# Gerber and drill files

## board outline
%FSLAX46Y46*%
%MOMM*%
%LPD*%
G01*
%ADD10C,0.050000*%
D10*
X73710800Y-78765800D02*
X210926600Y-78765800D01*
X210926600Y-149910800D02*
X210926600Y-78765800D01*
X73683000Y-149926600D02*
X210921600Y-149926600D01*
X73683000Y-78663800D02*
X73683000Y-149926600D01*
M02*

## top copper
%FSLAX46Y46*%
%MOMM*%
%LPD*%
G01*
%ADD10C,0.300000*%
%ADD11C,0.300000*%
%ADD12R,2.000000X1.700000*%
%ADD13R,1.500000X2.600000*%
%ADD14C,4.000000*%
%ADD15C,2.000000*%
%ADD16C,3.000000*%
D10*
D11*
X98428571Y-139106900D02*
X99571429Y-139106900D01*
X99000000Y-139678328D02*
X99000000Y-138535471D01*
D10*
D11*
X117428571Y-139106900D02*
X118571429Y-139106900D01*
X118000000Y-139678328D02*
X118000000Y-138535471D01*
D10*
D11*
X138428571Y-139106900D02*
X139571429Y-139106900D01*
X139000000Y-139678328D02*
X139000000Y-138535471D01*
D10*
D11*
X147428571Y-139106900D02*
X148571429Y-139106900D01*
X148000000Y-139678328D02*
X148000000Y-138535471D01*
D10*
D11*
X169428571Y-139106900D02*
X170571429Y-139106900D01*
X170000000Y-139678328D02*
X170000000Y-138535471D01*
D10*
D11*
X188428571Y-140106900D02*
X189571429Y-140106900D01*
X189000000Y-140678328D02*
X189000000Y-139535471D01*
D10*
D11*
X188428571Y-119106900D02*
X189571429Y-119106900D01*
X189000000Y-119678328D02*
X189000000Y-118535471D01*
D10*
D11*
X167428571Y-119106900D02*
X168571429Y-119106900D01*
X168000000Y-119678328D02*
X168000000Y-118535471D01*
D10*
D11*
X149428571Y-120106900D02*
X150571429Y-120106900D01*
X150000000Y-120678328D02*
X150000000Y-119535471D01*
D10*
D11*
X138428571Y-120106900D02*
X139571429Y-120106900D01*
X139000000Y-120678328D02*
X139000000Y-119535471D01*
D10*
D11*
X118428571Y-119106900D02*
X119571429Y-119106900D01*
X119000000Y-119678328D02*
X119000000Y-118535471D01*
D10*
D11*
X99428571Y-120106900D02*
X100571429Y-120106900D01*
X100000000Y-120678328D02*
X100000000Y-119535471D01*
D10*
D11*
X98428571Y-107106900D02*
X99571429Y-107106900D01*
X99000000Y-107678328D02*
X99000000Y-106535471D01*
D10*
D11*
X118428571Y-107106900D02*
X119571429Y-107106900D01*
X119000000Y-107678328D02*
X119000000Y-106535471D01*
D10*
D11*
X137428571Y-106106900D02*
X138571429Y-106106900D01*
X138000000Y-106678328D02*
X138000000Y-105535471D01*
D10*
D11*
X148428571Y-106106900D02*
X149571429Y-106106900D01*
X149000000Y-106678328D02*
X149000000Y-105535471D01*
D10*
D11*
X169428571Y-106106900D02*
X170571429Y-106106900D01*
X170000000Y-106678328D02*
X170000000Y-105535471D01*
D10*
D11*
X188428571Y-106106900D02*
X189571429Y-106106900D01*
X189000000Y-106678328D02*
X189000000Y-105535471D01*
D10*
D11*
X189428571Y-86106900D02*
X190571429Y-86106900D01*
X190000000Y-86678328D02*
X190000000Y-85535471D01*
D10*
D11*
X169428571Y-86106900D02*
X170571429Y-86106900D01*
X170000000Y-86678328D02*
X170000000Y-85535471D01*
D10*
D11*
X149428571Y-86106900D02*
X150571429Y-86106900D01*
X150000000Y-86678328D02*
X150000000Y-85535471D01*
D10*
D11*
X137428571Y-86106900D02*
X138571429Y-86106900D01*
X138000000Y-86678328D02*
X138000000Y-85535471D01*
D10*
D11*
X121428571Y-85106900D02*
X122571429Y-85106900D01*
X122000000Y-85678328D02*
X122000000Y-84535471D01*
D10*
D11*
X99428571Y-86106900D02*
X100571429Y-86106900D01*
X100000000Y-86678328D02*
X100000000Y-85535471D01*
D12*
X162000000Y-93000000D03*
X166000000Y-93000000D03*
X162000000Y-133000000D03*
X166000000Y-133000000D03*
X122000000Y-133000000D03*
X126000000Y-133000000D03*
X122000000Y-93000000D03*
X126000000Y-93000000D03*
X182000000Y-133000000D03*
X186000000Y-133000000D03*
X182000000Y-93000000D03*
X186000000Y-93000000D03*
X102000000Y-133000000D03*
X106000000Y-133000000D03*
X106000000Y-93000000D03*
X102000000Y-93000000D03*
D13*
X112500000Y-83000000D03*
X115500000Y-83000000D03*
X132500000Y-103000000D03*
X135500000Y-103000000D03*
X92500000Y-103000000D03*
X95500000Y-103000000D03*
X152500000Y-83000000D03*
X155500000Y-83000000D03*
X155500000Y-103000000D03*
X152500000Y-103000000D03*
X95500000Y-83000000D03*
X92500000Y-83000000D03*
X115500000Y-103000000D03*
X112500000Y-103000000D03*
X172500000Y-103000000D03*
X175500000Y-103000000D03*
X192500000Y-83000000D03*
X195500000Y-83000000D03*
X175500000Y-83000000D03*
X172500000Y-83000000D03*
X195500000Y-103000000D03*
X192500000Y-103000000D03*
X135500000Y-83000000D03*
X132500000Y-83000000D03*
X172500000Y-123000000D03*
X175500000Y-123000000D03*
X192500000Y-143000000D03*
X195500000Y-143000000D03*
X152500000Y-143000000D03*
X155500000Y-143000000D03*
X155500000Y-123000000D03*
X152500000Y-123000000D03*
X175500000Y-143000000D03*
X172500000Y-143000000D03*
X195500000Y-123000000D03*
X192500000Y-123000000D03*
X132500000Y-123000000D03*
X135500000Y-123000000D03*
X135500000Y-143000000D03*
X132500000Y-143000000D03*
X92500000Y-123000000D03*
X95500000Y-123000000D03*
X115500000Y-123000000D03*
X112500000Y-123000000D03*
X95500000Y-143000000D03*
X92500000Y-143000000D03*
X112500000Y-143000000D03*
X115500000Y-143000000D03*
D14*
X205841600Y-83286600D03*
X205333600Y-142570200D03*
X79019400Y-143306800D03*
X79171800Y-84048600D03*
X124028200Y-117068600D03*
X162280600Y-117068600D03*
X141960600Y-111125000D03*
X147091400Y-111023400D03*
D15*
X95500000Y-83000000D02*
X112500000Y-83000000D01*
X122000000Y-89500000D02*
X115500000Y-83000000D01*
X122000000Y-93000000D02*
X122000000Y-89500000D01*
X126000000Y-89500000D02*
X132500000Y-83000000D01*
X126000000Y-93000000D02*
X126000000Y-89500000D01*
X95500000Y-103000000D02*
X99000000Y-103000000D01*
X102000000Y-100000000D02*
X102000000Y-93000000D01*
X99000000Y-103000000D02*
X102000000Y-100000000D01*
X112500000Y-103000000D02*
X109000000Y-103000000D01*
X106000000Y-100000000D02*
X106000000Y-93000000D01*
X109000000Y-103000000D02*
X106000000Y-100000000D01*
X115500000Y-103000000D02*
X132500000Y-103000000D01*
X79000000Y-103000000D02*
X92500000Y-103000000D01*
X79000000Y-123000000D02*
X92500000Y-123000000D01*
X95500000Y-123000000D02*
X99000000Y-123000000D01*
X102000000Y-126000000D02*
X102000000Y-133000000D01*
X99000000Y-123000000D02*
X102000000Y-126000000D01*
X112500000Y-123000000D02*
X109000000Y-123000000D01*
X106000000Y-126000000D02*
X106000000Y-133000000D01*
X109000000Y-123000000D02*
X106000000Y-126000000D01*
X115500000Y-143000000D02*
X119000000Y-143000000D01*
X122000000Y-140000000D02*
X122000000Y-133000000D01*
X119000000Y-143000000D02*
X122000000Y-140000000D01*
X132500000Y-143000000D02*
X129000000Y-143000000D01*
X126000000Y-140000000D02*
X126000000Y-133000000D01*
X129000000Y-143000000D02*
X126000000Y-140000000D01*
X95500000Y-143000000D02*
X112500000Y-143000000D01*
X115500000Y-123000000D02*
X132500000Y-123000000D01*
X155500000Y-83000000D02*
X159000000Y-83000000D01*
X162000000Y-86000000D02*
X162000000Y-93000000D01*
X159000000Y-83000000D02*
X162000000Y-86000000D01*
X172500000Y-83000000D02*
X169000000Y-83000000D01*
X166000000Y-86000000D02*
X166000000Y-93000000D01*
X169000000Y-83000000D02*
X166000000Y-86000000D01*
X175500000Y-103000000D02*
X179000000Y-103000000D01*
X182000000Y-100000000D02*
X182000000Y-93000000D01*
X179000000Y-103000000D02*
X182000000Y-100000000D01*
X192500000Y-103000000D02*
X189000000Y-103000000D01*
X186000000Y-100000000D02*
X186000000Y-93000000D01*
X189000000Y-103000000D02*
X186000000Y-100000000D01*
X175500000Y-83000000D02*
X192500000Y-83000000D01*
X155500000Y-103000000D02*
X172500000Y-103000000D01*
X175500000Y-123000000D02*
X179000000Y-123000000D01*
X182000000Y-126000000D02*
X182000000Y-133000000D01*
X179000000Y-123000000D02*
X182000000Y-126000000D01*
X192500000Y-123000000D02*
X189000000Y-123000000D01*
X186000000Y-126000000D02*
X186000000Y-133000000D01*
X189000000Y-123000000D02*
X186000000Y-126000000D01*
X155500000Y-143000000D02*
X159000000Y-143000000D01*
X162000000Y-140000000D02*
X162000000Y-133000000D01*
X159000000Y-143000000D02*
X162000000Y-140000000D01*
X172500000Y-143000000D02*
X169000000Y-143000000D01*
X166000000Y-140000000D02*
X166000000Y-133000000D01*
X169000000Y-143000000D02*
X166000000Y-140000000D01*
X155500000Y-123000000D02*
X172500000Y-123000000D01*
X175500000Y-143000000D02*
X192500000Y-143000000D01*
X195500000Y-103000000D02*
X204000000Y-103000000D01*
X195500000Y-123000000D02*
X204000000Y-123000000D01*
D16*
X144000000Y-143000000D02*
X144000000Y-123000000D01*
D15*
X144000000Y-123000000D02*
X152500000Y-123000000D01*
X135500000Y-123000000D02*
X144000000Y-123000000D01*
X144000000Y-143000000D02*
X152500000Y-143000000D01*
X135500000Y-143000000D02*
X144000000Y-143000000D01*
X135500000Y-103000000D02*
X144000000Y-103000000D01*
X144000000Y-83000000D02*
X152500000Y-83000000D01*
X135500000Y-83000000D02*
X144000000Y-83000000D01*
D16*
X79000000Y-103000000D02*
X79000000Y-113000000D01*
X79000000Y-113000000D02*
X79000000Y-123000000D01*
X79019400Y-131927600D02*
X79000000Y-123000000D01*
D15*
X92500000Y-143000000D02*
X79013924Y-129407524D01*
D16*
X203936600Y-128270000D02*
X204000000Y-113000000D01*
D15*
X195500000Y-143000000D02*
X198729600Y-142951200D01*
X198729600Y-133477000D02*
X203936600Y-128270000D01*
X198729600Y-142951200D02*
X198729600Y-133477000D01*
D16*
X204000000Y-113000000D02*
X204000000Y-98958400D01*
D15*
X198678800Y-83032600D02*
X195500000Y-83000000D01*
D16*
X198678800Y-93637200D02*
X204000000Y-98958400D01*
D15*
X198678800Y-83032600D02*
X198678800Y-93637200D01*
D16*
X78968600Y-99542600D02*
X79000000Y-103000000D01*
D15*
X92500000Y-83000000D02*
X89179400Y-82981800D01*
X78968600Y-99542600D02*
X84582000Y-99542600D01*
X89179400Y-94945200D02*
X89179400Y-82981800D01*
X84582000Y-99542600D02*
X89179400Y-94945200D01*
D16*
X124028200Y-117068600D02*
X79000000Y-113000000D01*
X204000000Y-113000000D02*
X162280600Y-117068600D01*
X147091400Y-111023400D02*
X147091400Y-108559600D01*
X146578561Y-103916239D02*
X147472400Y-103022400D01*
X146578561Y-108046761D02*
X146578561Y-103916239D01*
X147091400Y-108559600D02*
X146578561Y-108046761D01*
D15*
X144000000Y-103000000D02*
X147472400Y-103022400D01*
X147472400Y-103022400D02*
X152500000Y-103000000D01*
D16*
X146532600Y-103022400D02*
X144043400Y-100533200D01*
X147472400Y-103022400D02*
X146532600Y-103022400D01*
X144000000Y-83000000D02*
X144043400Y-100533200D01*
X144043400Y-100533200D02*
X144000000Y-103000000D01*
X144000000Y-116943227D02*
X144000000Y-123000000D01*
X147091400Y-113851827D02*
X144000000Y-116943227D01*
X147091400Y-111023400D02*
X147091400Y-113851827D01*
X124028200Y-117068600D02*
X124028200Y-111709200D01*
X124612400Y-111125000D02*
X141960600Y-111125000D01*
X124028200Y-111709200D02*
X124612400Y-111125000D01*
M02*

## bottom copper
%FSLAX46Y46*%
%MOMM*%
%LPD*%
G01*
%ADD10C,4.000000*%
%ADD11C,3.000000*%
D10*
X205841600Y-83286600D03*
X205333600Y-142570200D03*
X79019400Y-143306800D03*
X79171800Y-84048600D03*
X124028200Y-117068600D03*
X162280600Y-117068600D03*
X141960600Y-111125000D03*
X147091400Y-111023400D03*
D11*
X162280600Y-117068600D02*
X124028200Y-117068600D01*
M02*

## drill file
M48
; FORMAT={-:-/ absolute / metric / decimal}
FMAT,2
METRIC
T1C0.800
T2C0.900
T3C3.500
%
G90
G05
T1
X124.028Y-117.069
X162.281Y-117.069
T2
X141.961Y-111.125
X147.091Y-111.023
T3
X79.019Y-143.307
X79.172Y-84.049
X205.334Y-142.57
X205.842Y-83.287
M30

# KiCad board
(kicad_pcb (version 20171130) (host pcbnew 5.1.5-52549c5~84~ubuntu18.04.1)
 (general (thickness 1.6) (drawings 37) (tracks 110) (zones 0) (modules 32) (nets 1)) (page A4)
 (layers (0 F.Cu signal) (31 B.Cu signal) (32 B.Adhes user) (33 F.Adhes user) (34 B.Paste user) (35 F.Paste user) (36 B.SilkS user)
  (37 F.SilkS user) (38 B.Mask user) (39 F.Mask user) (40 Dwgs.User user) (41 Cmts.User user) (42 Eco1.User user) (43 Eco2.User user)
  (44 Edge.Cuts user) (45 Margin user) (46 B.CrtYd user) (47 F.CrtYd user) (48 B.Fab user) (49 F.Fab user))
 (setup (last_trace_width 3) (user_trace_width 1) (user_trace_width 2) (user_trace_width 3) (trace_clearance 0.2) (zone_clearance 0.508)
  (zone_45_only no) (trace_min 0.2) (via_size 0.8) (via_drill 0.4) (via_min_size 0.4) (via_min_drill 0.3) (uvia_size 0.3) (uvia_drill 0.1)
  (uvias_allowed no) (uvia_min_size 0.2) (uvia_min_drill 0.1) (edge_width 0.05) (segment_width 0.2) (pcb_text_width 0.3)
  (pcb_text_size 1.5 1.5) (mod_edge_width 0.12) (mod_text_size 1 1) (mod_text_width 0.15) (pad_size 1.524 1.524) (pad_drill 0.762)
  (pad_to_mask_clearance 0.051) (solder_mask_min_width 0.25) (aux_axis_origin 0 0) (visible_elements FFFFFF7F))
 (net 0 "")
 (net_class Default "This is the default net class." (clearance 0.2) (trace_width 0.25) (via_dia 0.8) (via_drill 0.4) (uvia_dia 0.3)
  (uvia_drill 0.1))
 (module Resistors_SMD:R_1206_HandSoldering (layer F.Cu) (at 164 93)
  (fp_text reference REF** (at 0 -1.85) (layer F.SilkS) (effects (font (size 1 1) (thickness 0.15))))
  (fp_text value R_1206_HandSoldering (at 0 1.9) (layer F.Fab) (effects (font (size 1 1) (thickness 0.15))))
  (pad 1 smd rect (at -2 0) (size 2 1.7) (layers F.Cu F.Paste F.Mask))
  (pad 2 smd rect (at 2 0) (size 2 1.7) (layers F.Cu F.Paste F.Mask)))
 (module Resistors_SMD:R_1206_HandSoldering (layer F.Cu) (at 164 133)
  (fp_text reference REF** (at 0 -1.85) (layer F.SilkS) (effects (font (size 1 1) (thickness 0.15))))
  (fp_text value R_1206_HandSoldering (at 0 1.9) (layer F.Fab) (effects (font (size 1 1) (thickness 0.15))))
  (pad 1 smd rect (at -2 0) (size 2 1.7) (layers F.Cu F.Paste F.Mask))
  (pad 2 smd rect (at 2 0) (size 2 1.7) (layers F.Cu F.Paste F.Mask)))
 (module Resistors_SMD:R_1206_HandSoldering (layer F.Cu) (at 124 133)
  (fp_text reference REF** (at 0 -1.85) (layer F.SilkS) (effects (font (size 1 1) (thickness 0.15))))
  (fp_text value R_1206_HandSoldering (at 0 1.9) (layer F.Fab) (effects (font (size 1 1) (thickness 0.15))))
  (pad 1 smd rect (at -2 0) (size 2 1.7) (layers F.Cu F.Paste F.Mask))
  (pad 2 smd rect (at 2 0) (size 2 1.7) (layers F.Cu F.Paste F.Mask)))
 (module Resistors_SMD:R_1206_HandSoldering (layer F.Cu) (at 124 93)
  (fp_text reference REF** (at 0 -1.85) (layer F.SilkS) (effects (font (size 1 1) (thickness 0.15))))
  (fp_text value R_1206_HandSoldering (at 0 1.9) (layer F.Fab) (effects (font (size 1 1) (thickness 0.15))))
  (pad 1 smd rect (at -2 0) (size 2 1.7) (layers F.Cu F.Paste F.Mask))
  (pad 2 smd rect (at 2 0) (size 2 1.7) (layers F.Cu F.Paste F.Mask)))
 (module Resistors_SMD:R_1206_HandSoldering (layer F.Cu) (at 184 133)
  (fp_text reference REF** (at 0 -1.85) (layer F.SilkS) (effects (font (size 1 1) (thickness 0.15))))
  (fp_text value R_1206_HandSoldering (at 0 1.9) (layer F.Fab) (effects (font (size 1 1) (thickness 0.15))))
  (pad 1 smd rect (at -2 0) (size 2 1.7) (layers F.Cu F.Paste F.Mask))
  (pad 2 smd rect (at 2 0) (size 2 1.7) (layers F.Cu F.Paste F.Mask)))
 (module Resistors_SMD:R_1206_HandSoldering (layer F.Cu) (at 184 93)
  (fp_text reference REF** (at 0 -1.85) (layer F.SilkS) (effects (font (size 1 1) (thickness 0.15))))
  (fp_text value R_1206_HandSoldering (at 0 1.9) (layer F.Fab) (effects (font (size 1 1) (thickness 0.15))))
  (pad 1 smd rect (at -2 0) (size 2 1.7) (layers F.Cu F.Paste F.Mask))
  (pad 2 smd rect (at 2 0) (size 2 1.7) (layers F.Cu F.Paste F.Mask)))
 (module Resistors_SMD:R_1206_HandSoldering (layer F.Cu) (at 104 133)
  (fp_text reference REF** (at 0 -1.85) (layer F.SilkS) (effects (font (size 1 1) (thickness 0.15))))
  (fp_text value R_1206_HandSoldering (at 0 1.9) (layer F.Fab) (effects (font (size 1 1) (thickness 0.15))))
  (pad 1 smd rect (at -2 0) (size 2 1.7) (layers F.Cu F.Paste F.Mask))
  (pad 2 smd rect (at 2 0) (size 2 1.7) (layers F.Cu F.Paste F.Mask)))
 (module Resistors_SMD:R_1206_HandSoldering (layer F.Cu) (at 104 93)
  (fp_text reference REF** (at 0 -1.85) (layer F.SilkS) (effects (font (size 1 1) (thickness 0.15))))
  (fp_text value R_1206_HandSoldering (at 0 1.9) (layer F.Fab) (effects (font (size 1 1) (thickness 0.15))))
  (pad 2 smd rect (at 2 0) (size 2 1.7) (layers F.Cu F.Paste F.Mask))
  (pad 1 smd rect (at -2 0) (size 2 1.7) (layers F.Cu F.Paste F.Mask)))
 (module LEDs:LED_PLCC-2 (layer F.Cu) (at 114 83 180)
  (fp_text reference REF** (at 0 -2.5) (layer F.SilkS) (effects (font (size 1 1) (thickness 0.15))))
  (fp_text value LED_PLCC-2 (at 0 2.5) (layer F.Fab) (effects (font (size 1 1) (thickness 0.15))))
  (pad 2 smd rect (at 1.5 0 180) (size 1.5 2.6) (layers F.Cu F.Paste F.Mask))
  (pad 1 smd rect (at -1.5 0 180) (size 1.5 2.6) (layers F.Cu F.Paste F.Mask)))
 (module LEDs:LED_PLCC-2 (layer F.Cu) (at 134 103 180)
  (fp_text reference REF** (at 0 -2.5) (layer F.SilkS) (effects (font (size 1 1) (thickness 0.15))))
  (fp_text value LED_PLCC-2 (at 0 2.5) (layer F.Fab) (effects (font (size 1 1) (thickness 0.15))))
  (pad 2 smd rect (at 1.5 0 180) (size 1.5 2.6) (layers F.Cu F.Paste F.Mask))
  (pad 1 smd rect (at -1.5 0 180) (size 1.5 2.6) (layers F.Cu F.Paste F.Mask)))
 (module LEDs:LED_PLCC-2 (layer F.Cu) (at 94 103 180)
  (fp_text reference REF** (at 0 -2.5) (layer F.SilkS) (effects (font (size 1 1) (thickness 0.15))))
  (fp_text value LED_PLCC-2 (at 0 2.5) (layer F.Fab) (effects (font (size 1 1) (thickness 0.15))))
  (pad 2 smd rect (at 1.5 0 180) (size 1.5 2.6) (layers F.Cu F.Paste F.Mask))
  (pad 1 smd rect (at -1.5 0 180) (size 1.5 2.6) (layers F.Cu F.Paste F.Mask)))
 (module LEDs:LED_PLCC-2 (layer F.Cu) (at 154 83 180)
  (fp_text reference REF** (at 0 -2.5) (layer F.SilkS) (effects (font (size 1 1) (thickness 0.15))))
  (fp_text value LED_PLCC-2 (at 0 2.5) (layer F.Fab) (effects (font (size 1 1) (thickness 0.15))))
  (pad 2 smd rect (at 1.5 0 180) (size 1.5 2.6) (layers F.Cu F.Paste F.Mask))
  (pad 1 smd rect (at -1.5 0 180) (size 1.5 2.6) (layers F.Cu F.Paste F.Mask)))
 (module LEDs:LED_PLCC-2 (layer F.Cu) (at 154 103 180)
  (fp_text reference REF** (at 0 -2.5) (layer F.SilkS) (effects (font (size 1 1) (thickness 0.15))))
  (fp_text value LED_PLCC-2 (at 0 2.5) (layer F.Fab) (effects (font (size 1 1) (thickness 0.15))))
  (pad 1 smd rect (at -1.5 0 180) (size 1.5 2.6) (layers F.Cu F.Paste F.Mask))
  (pad 2 smd rect (at 1.5 0 180) (size 1.5 2.6) (layers F.Cu F.Paste F.Mask)))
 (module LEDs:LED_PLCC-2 (layer F.Cu) (at 94 83 180)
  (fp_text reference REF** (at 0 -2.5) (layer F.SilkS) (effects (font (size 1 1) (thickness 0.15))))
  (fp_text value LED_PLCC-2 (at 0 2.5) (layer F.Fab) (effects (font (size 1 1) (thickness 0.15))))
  (pad 1 smd rect (at -1.5 0 180) (size 1.5 2.6) (layers F.Cu F.Paste F.Mask))
  (pad 2 smd rect (at 1.5 0 180) (size 1.5 2.6) (layers F.Cu F.Paste F.Mask)))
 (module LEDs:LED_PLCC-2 (layer F.Cu) (at 114 103 180)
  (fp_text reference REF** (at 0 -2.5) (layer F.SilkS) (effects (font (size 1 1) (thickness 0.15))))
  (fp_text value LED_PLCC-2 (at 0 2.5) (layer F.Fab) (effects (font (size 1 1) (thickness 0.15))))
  (pad 1 smd rect (at -1.5 0 180) (size 1.5 2.6) (layers F.Cu F.Paste F.Mask))
  (pad 2 smd rect (at 1.5 0 180) (size 1.5 2.6) (layers F.Cu F.Paste F.Mask)))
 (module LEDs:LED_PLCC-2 (layer F.Cu) (at 174 103 180)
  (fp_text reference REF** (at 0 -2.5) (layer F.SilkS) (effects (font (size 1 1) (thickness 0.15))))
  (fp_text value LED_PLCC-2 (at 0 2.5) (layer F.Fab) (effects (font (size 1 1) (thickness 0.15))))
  (pad 2 smd rect (at 1.5 0 180) (size 1.5 2.6) (layers F.Cu F.Paste F.Mask))
  (pad 1 smd rect (at -1.5 0 180) (size 1.5 2.6) (layers F.Cu F.Paste F.Mask)))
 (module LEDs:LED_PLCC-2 (layer F.Cu) (at 194 83 180)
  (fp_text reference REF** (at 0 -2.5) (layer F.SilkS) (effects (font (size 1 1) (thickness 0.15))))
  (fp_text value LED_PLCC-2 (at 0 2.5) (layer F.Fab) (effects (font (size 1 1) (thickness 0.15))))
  (pad 2 smd rect (at 1.5 0 180) (size 1.5 2.6) (layers F.Cu F.Paste F.Mask))
  (pad 1 smd rect (at -1.5 0 180) (size 1.5 2.6) (layers F.Cu F.Paste F.Mask)))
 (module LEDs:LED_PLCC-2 (layer F.Cu) (at 174 83 180)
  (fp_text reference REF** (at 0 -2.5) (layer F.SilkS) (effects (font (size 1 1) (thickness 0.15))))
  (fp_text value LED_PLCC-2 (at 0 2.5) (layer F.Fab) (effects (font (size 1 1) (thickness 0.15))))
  (pad 1 smd rect (at -1.5 0 180) (size 1.5 2.6) (layers F.Cu F.Paste F.Mask))
  (pad 2 smd rect (at 1.5 0 180) (size 1.5 2.6) (layers F.Cu F.Paste F.Mask)))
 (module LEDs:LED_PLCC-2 (layer F.Cu) (at 194 103 180)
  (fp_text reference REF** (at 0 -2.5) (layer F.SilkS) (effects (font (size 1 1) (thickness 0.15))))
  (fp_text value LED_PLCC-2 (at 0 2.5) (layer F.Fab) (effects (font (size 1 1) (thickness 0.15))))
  (pad 1 smd rect (at -1.5 0 180) (size 1.5 2.6) (layers F.Cu F.Paste F.Mask))
  (pad 2 smd rect (at 1.5 0 180) (size 1.5 2.6) (layers F.Cu F.Paste F.Mask)))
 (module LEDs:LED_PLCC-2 (layer F.Cu) (at 134 83 180)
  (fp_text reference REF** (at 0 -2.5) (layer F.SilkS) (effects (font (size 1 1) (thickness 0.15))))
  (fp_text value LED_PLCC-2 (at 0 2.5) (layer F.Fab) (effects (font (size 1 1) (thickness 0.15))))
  (pad 1 smd rect (at -1.5 0 180) (size 1.5 2.6) (layers F.Cu F.Paste F.Mask))
  (pad 2 smd rect (at 1.5 0 180) (size 1.5 2.6) (layers F.Cu F.Paste F.Mask)))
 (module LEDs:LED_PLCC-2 (layer F.Cu) (at 174 123 180)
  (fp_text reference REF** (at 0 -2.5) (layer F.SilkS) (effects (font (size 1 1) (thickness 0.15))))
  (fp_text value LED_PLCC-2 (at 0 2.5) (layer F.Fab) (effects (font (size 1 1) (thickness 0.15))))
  (pad 2 smd rect (at 1.5 0 180) (size 1.5 2.6) (layers F.Cu F.Paste F.Mask))
  (pad 1 smd rect (at -1.5 0 180) (size 1.5 2.6) (layers F.Cu F.Paste F.Mask)))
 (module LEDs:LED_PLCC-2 (layer F.Cu) (at 194 143 180)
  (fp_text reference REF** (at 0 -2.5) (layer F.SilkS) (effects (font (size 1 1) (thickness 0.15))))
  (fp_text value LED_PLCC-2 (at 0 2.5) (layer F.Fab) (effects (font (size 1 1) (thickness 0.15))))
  (pad 2 smd rect (at 1.5 0 180) (size 1.5 2.6) (layers F.Cu F.Paste F.Mask))
  (pad 1 smd rect (at -1.5 0 180) (size 1.5 2.6) (layers F.Cu F.Paste F.Mask)))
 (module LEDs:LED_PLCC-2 (layer F.Cu) (at 154 143 180)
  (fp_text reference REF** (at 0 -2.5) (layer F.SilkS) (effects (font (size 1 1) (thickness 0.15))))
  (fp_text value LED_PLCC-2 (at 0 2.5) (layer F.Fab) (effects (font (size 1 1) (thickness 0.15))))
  (pad 2 smd rect (at 1.5 0 180) (size 1.5 2.6) (layers F.Cu F.Paste F.Mask))
  (pad 1 smd rect (at -1.5 0 180) (size 1.5 2.6) (layers F.Cu F.Paste F.Mask)))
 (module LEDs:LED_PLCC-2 (layer F.Cu) (at 154 123 180)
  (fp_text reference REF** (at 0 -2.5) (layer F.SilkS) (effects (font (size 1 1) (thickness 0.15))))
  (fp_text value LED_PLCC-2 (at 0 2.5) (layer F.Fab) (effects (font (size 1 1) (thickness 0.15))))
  (pad 1 smd rect (at -1.5 0 180) (size 1.5 2.6) (layers F.Cu F.Paste F.Mask))
  (pad 2 smd rect (at 1.5 0 180) (size 1.5 2.6) (layers F.Cu F.Paste F.Mask)))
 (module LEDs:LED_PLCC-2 (layer F.Cu) (at 174 143 180)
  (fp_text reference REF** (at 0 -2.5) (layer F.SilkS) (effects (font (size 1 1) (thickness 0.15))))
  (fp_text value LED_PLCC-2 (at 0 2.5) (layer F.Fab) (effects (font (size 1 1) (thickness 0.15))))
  (pad 1 smd rect (at -1.5 0 180) (size 1.5 2.6) (layers F.Cu F.Paste F.Mask))
  (pad 2 smd rect (at 1.5 0 180) (size 1.5 2.6) (layers F.Cu F.Paste F.Mask)))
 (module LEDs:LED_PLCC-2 (layer F.Cu) (at 194 123 180)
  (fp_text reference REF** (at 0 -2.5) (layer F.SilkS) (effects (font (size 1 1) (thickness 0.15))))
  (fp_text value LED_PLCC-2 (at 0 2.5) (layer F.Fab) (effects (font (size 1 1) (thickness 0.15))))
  (pad 1 smd rect (at -1.5 0 180) (size 1.5 2.6) (layers F.Cu F.Paste F.Mask))
  (pad 2 smd rect (at 1.5 0 180) (size 1.5 2.6) (layers F.Cu F.Paste F.Mask)))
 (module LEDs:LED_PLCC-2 (layer F.Cu) (at 134 123 180)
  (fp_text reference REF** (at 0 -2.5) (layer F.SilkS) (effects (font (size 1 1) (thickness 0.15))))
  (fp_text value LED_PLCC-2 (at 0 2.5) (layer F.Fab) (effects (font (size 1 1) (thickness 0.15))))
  (pad 2 smd rect (at 1.5 0 180) (size 1.5 2.6) (layers F.Cu F.Paste F.Mask))
  (pad 1 smd rect (at -1.5 0 180) (size 1.5 2.6) (layers F.Cu F.Paste F.Mask)))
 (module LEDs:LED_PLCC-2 (layer F.Cu) (at 134 143 180)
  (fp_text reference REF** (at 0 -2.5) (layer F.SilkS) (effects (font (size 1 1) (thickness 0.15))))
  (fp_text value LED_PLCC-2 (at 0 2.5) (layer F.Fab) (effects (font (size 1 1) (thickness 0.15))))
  (pad 1 smd rect (at -1.5 0 180) (size 1.5 2.6) (layers F.Cu F.Paste F.Mask))
  (pad 2 smd rect (at 1.5 0 180) (size 1.5 2.6) (layers F.Cu F.Paste F.Mask)))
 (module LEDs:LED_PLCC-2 (layer F.Cu) (at 94 123 180)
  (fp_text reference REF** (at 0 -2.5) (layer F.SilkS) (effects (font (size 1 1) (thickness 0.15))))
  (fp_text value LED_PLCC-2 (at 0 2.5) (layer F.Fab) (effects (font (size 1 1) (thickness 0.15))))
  (pad 2 smd rect (at 1.5 0 180) (size 1.5 2.6) (layers F.Cu F.Paste F.Mask))
  (pad 1 smd rect (at -1.5 0 180) (size 1.5 2.6) (layers F.Cu F.Paste F.Mask)))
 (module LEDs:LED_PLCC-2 (layer F.Cu) (at 114 123 180)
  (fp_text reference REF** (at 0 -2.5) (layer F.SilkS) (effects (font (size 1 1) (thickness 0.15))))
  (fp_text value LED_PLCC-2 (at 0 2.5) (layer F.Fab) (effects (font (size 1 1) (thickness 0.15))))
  (pad 1 smd rect (at -1.5 0 180) (size 1.5 2.6) (layers F.Cu F.Paste F.Mask))
  (pad 2 smd rect (at 1.5 0 180) (size 1.5 2.6) (layers F.Cu F.Paste F.Mask)))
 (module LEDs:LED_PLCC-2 (layer F.Cu) (at 94 143 180)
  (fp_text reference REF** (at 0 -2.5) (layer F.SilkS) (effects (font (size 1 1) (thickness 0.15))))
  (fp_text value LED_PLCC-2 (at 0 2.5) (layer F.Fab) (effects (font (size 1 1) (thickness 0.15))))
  (pad 1 smd rect (at -1.5 0 180) (size 1.5 2.6) (layers F.Cu F.Paste F.Mask))
  (pad 2 smd rect (at 1.5 0 180) (size 1.5 2.6) (layers F.Cu F.Paste F.Mask)))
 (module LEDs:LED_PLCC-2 (layer F.Cu) (at 114 143 180)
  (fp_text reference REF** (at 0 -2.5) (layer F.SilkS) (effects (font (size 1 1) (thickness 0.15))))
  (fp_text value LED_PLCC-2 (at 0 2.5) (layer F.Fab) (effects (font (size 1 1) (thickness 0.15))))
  (pad 2 smd rect (at 1.5 0 180) (size 1.5 2.6) (layers F.Cu F.Paste F.Mask))
  (pad 1 smd rect (at -1.5 0 180) (size 1.5 2.6) (layers F.Cu F.Paste F.Mask)))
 (gr_line (start 73.7108 78.7658) (end 210.9266 78.7658) (layer Edge.Cuts) (width 0.05))
 (gr_line (start 210.9266 149.9108) (end 210.9266 78.7658) (layer Edge.Cuts) (width 0.05))
 (gr_line (start 73.683 149.9266) (end 210.9216 149.9266) (layer Edge.Cuts) (width 0.05))
 (gr_line (start 73.683 78.6638) (end 73.683 149.9266) (layer Edge.Cuts) (width 0.05))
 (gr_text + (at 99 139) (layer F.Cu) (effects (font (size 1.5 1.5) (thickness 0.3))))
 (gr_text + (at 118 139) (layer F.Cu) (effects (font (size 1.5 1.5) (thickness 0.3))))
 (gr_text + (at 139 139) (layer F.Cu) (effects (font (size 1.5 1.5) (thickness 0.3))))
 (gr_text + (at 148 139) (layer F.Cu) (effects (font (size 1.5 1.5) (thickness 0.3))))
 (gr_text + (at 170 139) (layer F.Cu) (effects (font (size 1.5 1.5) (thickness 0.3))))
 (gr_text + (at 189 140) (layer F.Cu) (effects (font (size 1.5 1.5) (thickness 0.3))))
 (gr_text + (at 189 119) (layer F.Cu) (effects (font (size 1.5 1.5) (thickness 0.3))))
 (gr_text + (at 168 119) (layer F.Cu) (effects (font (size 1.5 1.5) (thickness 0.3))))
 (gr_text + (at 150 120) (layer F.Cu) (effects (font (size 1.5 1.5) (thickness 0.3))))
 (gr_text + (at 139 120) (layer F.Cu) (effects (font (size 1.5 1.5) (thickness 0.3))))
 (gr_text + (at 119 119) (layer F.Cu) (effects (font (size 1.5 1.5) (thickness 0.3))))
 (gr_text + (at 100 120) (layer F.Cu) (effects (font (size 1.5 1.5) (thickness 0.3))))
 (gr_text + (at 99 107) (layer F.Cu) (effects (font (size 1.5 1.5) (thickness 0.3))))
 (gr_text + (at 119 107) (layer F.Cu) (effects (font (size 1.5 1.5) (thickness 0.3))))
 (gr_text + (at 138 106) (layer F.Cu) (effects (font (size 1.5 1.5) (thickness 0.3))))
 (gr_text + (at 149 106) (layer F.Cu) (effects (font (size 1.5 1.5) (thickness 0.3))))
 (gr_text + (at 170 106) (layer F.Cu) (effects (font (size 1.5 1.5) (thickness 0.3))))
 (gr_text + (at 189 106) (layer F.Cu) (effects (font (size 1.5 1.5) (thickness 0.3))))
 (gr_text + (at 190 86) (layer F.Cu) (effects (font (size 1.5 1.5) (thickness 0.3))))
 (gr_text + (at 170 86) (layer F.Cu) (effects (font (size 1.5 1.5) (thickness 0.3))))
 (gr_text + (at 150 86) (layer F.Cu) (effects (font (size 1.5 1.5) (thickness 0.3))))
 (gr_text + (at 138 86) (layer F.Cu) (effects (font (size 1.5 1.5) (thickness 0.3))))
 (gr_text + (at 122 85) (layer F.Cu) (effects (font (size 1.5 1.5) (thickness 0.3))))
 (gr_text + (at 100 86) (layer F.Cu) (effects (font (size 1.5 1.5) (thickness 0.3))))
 (segment (start 95.5 83) (end 112.5 83) (width 2) (layer F.Cu) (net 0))
 (segment (start 122 89.5) (end 115.5 83) (width 2) (layer F.Cu) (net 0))
 (segment (start 122 93) (end 122 89.5) (width 2) (layer F.Cu) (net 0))
 (segment (start 126 89.5) (end 132.5 83) (width 2) (layer F.Cu) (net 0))
 (segment (start 126 93) (end 126 89.5) (width 2) (layer F.Cu) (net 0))
 (segment (start 95.5 103) (end 99 103) (width 2) (layer F.Cu) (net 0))
 (segment (start 102 100) (end 102 93) (width 2) (layer F.Cu) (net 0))
 (segment (start 99 103) (end 102 100) (width 2) (layer F.Cu) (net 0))
 (segment (start 112.5 103) (end 109 103) (width 2) (layer F.Cu) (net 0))
 (segment (start 106 100) (end 106 93) (width 2) (layer F.Cu) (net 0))
 (segment (start 109 103) (end 106 100) (width 2) (layer F.Cu) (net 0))
 (segment (start 115.5 103) (end 132.5 103) (width 2) (layer F.Cu) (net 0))
 (segment (start 79 103) (end 92.5 103) (width 2) (layer F.Cu) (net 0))
 (segment (start 79 123) (end 92.5 123) (width 2) (layer F.Cu) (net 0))
 (segment (start 95.5 123) (end 99 123) (width 2) (layer F.Cu) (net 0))
 (segment (start 102 126) (end 102 133) (width 2) (layer F.Cu) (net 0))
 (segment (start 99 123) (end 102 126) (width 2) (layer F.Cu) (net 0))
 (segment (start 112.5 123) (end 109 123) (width 2) (layer F.Cu) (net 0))
 (segment (start 106 126) (end 106 133) (width 2) (layer F.Cu) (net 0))
 (segment (start 109 123) (end 106 126) (width 2) (layer F.Cu) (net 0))
 (segment (start 115.5 143) (end 119 143) (width 2) (layer F.Cu) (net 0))
 (segment (start 122 140) (end 122 133) (width 2) (layer F.Cu) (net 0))
 (segment (start 119 143) (end 122 140) (width 2) (layer F.Cu) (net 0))
 (segment (start 132.5 143) (end 129 143) (width 2) (layer F.Cu) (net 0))
 (segment (start 126 140) (end 126 133) (width 2) (layer F.Cu) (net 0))
 (segment (start 129 143) (end 126 140) (width 2) (layer F.Cu) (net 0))
 (segment (start 95.5 143) (end 112.5 143) (width 2) (layer F.Cu) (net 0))
 (segment (start 115.5 123) (end 132.5 123) (width 2) (layer F.Cu) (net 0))
 (segment (start 155.5 83) (end 159 83) (width 2) (layer F.Cu) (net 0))
 (segment (start 162 86) (end 162 93) (width 2) (layer F.Cu) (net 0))
 (segment (start 159 83) (end 162 86) (width 2) (layer F.Cu) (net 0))
 (segment (start 172.5 83) (end 169 83) (width 2) (layer F.Cu) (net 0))
 (segment (start 166 86) (end 166 93) (width 2) (layer F.Cu) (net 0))
 (segment (start 169 83) (end 166 86) (width 2) (layer F.Cu) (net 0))
 (segment (start 175.5 103) (end 179 103) (width 2) (layer F.Cu) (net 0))
 (segment (start 182 100) (end 182 93) (width 2) (layer F.Cu) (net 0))
 (segment (start 179 103) (end 182 100) (width 2) (layer F.Cu) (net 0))
 (segment (start 192.5 103) (end 189 103) (width 2) (layer F.Cu) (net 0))
 (segment (start 186 100) (end 186 93) (width 2) (layer F.Cu) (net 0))
 (segment (start 189 103) (end 186 100) (width 2) (layer F.Cu) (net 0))
 (segment (start 175.5 83) (end 192.5 83) (width 2) (layer F.Cu) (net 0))
 (segment (start 155.5 103) (end 172.5 103) (width 2) (layer F.Cu) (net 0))
 (segment (start 175.5 123) (end 179 123) (width 2) (layer F.Cu) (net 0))
 (segment (start 182 126) (end 182 133) (width 2) (layer F.Cu) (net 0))
 (segment (start 179 123) (end 182 126) (width 2) (layer F.Cu) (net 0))
 (segment (start 192.5 123) (end 189 123) (width 2) (layer F.Cu) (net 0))
 (segment (start 186 126) (end 186 133) (width 2) (layer F.Cu) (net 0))
 (segment (start 189 123) (end 186 126) (width 2) (layer F.Cu) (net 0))
 (segment (start 155.5 143) (end 159 143) (width 2) (layer F.Cu) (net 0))
 (segment (start 162 140) (end 162 133) (width 2) (layer F.Cu) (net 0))
 (segment (start 159 143) (end 162 140) (width 2) (layer F.Cu) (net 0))
 (segment (start 172.5 143) (end 169 143) (width 2) (layer F.Cu) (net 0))
 (segment (start 166 140) (end 166 133) (width 2) (layer F.Cu) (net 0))
 (segment (start 169 143) (end 166 140) (width 2) (layer F.Cu) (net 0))
 (segment (start 155.5 123) (end 172.5 123) (width 2) (layer F.Cu) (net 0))
 (segment (start 175.5 143) (end 192.5 143) (width 2) (layer F.Cu) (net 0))
 (segment (start 195.5 103) (end 204 103) (width 2) (layer F.Cu) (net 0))
 (segment (start 195.5 123) (end 204 123) (width 2) (layer F.Cu) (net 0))
 (segment (start 144 143) (end 144 123) (width 3) (layer F.Cu) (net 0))
 (segment (start 144 123) (end 152.5 123) (width 2) (layer F.Cu) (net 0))
 (segment (start 135.5 123) (end 144 123) (width 2) (layer F.Cu) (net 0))
 (segment (start 144 143) (end 152.5 143) (width 2) (layer F.Cu) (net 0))
 (segment (start 135.5 143) (end 144 143) (width 2) (layer F.Cu) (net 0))
 (segment (start 135.5 103) (end 144 103) (width 2) (layer F.Cu) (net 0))
 (segment (start 144 83) (end 152.5 83) (width 2) (layer F.Cu) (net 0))
 (segment (start 135.5 83) (end 144 83) (width 2) (layer F.Cu) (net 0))
 (segment (start 79 103) (end 79 113) (width 3) (layer F.Cu) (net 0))
 (segment (start 79 113) (end 79 123) (width 3) (layer F.Cu) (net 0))
 (via (at 205.8416 83.2866) (size 4) (drill 3.5) (layers F.Cu B.Cu) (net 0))
 (via (at 205.3336 142.5702) (size 4) (drill 3.5) (layers F.Cu B.Cu) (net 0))
 (segment (start 79.0194 131.9276) (end 79 123) (width 3) (layer F.Cu) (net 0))
 (segment (start 92.5 143) (end 79.013924 129.407524) (width 2) (layer F.Cu) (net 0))
 (segment (start 203.9366 128.27) (end 204 113) (width 3) (layer F.Cu) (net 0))
 (segment (start 195.5 143) (end 198.7296 142.9512) (width 2) (layer F.Cu) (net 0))
 (segment (start 198.7296 133.477) (end 203.9366 128.27) (width 2) (layer F.Cu) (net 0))
 (segment (start 198.7296 142.9512) (end 198.7296 133.477) (width 2) (layer F.Cu) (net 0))
 (segment (start 204 113) (end 204 98.9584) (width 3) (layer F.Cu) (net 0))
 (segment (start 198.6788 83.0326) (end 195.5 83) (width 2) (layer F.Cu) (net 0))
 (segment (start 198.6788 93.6372) (end 204 98.9584) (width 3) (layer F.Cu) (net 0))
 (segment (start 198.6788 83.0326) (end 198.6788 93.6372) (width 2) (layer F.Cu) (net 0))
 (segment (start 78.9686 99.5426) (end 79 103) (width 3) (layer F.Cu) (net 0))
 (segment (start 92.5 83) (end 89.1794 82.9818) (width 2) (layer F.Cu) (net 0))
 (segment (start 78.9686 99.5426) (end 84.582 99.5426) (width 2) (layer F.Cu) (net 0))
 (segment (start 89.1794 94.9452) (end 89.1794 82.9818) (width 2) (layer F.Cu) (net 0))
 (segment (start 84.582 99.5426) (end 89.1794 94.9452) (width 2) (layer F.Cu) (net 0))
 (via (at 79.0194 143.3068) (size 4) (drill 3.5) (layers F.Cu B.Cu) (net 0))
 (via (at 79.1718 84.0486) (size 4) (drill 3.5) (layers F.Cu B.Cu) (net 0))
 (segment (start 124.0282 117.0686) (end 79 113) (width 3) (layer F.Cu) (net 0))
 (via (at 124.0282 117.0686) (size 4) (drill 0.8) (layers F.Cu B.Cu) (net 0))
 (segment (start 162.2806 117.0686) (end 124.0282 117.0686) (width 3) (layer B.Cu) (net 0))
 (via (at 162.2806 117.0686) (size 4) (drill 0.8) (layers F.Cu B.Cu) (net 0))
 (segment (start 204 113) (end 162.2806 117.0686) (width 3) (layer F.Cu) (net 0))
 (via (at 141.9606 111.125) (size 4) (drill 0.9) (layers F.Cu B.Cu) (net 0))
 (via (at 147.0914 111.0234) (size 4) (drill 0.9) (layers F.Cu B.Cu) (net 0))
 (segment (start 147.0914 111.0234) (end 147.0914 108.5596) (width 3) (layer F.Cu) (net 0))
 (segment (start 146.578561 103.916239) (end 147.4724 103.0224) (width 3) (layer F.Cu) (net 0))
 (segment (start 146.578561 108.046761) (end 146.578561 103.916239) (width 3) (layer F.Cu) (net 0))
 (segment (start 147.0914 108.5596) (end 146.578561 108.046761) (width 3) (layer F.Cu) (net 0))
 (segment (start 144 103) (end 147.4724 103.0224) (width 2) (layer F.Cu) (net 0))
 (segment (start 147.4724 103.0224) (end 152.5 103) (width 2) (layer F.Cu) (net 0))
 (segment (start 146.5326 103.0224) (end 144.0434 100.5332) (width 3) (layer F.Cu) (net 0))
 (segment (start 147.4724 103.0224) (end 146.5326 103.0224) (width 3) (layer F.Cu) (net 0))
 (segment (start 144 83) (end 144.0434 100.5332) (width 3) (layer F.Cu) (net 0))
 (segment (start 144.0434 100.5332) (end 144 103) (width 3) (layer F.Cu) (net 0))
 (segment (start 144 116.943227) (end 144 123) (width 3) (layer F.Cu) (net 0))
 (segment (start 147.0914 113.851827) (end 144 116.943227) (width 3) (layer F.Cu) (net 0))
 (segment (start 147.0914 111.0234) (end 147.0914 113.851827) (width 3) (layer F.Cu) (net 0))
 (segment (start 124.0282 117.0686) (end 124.0282 111.7092) (width 3) (layer F.Cu) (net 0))
 (segment (start 124.6124 111.125) (end 141.9606 111.125) (width 3) (layer F.Cu) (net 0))
 (segment (start 124.0282 111.7092) (end 124.6124 111.125) (width 3) (layer F.Cu) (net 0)))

